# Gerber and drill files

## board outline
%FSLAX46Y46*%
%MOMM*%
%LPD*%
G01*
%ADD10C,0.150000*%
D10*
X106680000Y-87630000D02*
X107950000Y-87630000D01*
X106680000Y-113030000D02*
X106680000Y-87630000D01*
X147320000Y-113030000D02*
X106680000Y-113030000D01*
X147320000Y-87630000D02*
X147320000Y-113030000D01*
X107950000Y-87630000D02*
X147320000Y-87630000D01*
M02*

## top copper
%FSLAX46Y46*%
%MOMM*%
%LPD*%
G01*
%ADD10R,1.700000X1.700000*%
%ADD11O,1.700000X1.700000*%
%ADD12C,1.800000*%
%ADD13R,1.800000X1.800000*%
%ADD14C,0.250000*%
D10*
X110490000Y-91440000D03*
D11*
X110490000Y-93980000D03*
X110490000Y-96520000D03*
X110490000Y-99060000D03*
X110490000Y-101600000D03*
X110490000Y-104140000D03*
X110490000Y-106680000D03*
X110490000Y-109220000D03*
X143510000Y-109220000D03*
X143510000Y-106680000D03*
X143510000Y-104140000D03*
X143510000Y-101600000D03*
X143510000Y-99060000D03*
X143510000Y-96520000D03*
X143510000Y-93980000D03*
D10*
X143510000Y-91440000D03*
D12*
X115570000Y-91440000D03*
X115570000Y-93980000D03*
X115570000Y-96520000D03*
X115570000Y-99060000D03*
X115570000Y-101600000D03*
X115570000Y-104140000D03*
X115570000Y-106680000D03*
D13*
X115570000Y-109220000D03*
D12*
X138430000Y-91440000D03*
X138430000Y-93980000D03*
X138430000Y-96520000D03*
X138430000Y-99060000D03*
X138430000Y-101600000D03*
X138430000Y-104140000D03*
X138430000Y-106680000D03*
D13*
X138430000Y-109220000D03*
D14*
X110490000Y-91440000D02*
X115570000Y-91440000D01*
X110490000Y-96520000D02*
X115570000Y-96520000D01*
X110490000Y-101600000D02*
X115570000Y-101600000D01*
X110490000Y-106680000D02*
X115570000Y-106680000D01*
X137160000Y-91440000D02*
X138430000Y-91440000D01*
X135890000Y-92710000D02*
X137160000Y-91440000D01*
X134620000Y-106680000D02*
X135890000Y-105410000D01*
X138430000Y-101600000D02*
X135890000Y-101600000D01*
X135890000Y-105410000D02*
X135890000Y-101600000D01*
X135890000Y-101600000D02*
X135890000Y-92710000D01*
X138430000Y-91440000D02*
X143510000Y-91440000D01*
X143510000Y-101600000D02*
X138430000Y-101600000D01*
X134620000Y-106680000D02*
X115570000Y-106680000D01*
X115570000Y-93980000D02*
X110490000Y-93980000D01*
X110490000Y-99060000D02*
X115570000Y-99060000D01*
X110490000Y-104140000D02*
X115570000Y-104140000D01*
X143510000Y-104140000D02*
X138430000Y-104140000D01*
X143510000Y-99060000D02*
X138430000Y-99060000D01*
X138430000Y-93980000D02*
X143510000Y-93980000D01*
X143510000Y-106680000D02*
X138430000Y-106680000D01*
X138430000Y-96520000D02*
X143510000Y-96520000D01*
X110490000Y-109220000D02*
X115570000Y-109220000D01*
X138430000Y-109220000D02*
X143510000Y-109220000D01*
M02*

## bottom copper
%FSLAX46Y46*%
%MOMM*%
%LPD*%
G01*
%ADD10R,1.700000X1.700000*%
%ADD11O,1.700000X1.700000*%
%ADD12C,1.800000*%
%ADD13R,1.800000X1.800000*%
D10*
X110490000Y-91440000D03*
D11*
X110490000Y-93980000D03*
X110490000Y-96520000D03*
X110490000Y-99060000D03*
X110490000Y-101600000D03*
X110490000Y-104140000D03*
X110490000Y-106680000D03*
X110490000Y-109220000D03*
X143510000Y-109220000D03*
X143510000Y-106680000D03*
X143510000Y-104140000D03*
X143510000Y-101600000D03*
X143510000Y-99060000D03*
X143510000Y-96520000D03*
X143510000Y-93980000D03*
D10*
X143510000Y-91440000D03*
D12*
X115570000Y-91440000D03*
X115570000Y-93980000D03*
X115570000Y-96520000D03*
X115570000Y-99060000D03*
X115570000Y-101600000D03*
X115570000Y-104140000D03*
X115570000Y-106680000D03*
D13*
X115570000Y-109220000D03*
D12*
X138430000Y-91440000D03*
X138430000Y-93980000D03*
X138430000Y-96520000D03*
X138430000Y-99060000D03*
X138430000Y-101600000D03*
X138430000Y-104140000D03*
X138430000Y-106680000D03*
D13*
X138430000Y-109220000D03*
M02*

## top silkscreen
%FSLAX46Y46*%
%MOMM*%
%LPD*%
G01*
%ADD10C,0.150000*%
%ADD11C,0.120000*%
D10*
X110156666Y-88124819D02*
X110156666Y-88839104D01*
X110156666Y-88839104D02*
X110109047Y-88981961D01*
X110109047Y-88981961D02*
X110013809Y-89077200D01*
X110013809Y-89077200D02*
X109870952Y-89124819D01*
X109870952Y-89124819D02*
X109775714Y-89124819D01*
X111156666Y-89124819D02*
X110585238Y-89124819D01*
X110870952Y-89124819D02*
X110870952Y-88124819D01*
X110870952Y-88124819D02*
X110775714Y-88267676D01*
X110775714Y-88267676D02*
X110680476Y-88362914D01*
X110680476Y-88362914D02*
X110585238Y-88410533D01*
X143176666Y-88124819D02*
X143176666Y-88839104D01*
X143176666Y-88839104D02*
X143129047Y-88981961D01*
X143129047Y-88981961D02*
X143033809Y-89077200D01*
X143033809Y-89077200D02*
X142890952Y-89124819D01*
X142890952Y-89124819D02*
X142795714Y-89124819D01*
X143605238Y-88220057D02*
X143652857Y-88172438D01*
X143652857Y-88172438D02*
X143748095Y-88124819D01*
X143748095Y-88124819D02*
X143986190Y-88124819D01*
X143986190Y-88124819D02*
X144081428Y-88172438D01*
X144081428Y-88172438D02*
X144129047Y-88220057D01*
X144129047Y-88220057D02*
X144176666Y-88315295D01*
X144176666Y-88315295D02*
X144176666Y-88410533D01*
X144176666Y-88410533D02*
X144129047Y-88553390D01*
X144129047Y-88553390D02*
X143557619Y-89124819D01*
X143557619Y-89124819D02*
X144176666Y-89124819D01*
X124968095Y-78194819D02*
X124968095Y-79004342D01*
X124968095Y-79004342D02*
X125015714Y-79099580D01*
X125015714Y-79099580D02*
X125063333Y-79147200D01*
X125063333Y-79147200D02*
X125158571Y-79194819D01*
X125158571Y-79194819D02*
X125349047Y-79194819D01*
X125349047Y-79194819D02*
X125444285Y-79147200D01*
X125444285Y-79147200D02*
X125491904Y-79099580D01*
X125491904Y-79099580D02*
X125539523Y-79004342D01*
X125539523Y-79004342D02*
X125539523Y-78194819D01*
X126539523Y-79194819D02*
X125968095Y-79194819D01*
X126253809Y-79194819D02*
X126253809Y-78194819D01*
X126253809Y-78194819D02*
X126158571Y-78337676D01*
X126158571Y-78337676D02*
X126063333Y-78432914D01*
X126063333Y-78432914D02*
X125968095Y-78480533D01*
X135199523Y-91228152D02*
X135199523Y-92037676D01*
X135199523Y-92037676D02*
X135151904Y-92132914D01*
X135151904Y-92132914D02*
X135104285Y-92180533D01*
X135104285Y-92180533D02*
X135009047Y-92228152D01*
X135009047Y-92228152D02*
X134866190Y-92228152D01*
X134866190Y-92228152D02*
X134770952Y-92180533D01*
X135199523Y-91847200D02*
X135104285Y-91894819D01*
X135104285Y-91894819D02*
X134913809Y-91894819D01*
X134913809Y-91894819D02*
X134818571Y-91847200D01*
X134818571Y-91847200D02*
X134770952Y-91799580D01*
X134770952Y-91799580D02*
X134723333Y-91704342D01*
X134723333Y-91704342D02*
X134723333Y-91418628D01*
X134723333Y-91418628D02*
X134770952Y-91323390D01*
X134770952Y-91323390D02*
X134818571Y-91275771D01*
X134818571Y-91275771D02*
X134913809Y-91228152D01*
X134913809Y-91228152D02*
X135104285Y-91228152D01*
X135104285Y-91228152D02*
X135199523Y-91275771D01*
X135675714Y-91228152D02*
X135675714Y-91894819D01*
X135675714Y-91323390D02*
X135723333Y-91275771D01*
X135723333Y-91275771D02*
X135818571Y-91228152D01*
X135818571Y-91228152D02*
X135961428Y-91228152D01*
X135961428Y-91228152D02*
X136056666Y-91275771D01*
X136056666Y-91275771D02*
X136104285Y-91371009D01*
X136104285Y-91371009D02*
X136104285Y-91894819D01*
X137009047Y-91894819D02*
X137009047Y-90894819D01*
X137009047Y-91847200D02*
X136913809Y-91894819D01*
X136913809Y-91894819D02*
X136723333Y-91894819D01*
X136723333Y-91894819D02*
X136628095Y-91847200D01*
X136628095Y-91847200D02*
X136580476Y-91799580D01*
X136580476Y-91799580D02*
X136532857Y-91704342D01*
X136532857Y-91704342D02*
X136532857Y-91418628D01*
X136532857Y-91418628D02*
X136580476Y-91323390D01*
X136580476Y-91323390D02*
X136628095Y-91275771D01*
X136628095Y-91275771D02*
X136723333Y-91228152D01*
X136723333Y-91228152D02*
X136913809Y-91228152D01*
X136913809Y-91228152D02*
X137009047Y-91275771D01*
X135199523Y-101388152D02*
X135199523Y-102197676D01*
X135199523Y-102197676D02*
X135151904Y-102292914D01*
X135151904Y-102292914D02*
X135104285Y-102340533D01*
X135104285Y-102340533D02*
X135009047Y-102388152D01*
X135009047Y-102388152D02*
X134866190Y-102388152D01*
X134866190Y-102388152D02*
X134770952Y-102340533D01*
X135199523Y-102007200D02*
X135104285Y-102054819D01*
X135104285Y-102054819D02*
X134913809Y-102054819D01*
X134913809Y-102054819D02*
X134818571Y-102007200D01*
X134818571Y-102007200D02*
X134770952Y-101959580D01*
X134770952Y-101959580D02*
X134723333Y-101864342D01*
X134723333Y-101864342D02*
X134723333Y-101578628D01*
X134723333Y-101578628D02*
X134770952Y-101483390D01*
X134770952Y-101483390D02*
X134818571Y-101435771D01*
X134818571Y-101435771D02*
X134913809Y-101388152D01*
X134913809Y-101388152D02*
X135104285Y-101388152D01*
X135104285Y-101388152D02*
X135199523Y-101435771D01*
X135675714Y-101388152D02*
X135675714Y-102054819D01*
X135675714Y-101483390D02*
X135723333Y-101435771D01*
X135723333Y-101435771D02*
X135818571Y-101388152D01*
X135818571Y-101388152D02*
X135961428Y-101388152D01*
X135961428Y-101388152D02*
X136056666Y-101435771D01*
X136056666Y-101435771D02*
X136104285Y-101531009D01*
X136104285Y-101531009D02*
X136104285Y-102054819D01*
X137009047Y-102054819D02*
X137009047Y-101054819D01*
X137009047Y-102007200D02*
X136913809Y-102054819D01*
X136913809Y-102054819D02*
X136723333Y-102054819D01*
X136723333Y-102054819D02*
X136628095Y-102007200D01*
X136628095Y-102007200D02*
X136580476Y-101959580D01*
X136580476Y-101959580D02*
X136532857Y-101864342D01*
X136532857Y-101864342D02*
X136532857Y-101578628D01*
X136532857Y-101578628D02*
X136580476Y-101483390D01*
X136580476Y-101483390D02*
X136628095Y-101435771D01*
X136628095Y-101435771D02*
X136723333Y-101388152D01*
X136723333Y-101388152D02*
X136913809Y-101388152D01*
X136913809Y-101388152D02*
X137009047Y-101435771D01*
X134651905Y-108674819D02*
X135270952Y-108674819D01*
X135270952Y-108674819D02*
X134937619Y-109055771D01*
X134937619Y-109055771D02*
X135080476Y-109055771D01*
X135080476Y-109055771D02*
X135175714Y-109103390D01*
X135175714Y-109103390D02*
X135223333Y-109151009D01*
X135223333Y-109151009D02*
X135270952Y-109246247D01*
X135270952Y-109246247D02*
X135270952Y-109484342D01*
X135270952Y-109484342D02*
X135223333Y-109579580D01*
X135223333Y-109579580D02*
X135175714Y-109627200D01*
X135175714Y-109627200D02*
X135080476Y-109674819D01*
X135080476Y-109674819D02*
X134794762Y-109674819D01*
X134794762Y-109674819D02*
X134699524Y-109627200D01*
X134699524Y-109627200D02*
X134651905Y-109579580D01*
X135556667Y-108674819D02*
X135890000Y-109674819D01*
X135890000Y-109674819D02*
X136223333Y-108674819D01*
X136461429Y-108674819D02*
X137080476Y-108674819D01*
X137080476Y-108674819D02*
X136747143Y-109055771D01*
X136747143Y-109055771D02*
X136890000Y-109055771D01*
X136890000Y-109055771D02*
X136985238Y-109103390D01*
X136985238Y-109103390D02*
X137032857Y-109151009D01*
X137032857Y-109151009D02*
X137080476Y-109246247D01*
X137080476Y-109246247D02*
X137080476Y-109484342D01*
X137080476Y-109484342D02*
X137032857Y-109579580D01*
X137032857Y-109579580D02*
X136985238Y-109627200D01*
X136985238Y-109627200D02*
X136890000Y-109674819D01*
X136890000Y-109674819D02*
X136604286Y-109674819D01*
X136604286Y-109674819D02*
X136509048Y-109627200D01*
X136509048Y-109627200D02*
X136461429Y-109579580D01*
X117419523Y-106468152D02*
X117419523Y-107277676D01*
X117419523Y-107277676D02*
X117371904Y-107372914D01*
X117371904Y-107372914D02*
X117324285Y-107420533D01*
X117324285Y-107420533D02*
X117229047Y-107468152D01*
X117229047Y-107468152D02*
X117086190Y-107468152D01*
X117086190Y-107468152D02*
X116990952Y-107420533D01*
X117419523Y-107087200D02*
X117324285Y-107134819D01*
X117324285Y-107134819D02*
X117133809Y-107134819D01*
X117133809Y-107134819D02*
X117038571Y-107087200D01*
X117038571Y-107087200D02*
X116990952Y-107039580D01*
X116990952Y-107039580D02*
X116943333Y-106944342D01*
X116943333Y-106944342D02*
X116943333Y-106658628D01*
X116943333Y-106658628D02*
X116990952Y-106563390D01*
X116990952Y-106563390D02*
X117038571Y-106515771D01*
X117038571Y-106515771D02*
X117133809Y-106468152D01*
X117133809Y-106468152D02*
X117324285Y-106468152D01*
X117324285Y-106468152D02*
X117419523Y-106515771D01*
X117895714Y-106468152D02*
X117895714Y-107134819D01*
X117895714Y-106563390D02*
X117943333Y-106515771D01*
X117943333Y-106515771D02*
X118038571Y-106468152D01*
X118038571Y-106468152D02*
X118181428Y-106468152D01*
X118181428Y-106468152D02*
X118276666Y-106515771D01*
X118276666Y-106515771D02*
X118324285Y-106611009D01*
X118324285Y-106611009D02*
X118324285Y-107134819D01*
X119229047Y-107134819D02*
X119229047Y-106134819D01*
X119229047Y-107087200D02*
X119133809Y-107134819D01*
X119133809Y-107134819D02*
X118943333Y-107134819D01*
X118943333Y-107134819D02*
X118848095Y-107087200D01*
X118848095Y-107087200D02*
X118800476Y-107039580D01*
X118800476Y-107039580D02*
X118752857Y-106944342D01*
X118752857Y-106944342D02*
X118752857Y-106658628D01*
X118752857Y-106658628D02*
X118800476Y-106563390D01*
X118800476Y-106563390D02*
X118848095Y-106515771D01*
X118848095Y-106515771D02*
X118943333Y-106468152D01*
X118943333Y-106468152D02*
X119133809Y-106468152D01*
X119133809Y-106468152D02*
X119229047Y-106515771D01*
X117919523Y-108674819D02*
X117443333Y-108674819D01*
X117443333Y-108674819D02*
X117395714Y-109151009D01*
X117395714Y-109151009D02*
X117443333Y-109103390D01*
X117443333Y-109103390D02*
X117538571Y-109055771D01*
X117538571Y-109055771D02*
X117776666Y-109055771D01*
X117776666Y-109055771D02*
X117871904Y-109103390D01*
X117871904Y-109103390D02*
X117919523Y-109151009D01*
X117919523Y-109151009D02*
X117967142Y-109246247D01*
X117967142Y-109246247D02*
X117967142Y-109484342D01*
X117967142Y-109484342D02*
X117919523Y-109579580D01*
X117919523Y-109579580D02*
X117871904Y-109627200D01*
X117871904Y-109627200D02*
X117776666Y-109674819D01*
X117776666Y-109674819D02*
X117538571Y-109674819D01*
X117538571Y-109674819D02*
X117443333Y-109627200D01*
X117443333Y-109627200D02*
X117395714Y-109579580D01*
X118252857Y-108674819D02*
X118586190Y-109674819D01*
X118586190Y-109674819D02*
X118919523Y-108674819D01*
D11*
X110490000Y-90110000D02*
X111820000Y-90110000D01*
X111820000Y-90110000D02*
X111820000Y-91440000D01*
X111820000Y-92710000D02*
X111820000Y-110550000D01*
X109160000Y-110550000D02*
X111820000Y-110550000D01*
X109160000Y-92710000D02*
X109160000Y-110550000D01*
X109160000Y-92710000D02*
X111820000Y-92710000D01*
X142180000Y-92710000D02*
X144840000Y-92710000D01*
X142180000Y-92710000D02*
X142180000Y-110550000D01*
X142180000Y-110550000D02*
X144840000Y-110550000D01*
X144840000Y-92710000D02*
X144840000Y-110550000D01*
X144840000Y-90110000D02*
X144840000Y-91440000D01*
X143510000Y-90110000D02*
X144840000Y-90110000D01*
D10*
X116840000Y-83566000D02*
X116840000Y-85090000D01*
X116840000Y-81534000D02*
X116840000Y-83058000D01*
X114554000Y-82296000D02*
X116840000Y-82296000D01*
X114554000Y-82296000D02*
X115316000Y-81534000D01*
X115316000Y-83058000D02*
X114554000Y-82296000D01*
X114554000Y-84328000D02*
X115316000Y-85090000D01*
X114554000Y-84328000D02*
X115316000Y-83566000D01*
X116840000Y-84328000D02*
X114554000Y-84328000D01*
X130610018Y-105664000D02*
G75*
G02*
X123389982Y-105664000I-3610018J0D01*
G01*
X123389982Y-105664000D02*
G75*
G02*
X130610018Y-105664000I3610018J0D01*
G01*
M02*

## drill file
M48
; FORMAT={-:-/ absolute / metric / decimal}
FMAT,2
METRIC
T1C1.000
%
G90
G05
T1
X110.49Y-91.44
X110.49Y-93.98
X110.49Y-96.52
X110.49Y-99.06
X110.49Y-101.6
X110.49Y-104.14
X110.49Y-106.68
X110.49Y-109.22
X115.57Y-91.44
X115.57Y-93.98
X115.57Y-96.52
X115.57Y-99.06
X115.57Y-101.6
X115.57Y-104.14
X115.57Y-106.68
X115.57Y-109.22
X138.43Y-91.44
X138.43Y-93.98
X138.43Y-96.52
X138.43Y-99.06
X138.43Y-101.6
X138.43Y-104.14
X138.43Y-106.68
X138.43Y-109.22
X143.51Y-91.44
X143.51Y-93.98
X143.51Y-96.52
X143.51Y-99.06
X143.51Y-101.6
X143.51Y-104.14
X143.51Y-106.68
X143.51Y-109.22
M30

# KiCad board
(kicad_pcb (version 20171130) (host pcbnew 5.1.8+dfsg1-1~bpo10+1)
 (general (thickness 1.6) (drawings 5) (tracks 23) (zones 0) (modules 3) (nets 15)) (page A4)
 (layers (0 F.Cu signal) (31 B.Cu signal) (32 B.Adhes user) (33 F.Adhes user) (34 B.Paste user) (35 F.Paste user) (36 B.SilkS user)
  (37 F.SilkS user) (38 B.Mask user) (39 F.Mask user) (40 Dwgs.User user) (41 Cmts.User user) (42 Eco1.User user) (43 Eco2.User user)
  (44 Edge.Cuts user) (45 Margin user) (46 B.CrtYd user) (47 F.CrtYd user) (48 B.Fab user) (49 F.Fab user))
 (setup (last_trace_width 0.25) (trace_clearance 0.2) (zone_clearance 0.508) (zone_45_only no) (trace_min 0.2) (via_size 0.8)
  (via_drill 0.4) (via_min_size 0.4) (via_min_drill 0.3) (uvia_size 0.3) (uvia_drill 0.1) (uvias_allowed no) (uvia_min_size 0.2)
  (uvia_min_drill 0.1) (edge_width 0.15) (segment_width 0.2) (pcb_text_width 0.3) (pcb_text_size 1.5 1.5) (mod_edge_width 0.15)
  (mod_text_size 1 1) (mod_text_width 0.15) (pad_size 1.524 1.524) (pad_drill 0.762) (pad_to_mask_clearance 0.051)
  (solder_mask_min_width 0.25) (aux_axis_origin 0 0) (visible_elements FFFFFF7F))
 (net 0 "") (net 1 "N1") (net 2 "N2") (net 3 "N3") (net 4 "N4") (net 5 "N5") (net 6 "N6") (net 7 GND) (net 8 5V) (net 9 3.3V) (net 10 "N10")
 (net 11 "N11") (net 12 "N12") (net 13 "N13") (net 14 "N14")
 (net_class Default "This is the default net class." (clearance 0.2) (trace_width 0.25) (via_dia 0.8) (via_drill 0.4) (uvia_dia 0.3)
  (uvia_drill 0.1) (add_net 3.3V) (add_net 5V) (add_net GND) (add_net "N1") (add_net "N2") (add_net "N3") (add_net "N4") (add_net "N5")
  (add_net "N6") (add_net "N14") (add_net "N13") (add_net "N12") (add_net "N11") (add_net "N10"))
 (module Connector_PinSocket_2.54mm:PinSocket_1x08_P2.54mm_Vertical (layer F.Cu) (at 110.49 91.44)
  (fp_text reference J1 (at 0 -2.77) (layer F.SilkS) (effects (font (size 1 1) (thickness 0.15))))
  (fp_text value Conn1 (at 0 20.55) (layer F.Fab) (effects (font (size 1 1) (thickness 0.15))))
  (fp_line (start 0 -1.33) (end 1.33 -1.33) (layer F.SilkS) (width 0.12))
  (fp_line (start 1.33 -1.33) (end 1.33 0) (layer F.SilkS) (width 0.12))
  (fp_line (start 1.33 1.27) (end 1.33 19.11) (layer F.SilkS) (width 0.12))
  (fp_line (start -1.33 19.11) (end 1.33 19.11) (layer F.SilkS) (width 0.12))
  (fp_line (start -1.33 1.27) (end -1.33 19.11) (layer F.SilkS) (width 0.12))
  (fp_line (start -1.33 1.27) (end 1.33 1.27) (layer F.SilkS) (width 0.12))
  (pad 1 thru_hole rect (at 0 0) (size 1.7 1.7) (drill 1) (layers *.Cu *.Mask) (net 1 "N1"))
  (pad 2 thru_hole oval (at 0 2.54) (size 1.7 1.7) (drill 1) (layers *.Cu *.Mask) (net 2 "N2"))
  (pad 3 thru_hole oval (at 0 5.08) (size 1.7 1.7) (drill 1) (layers *.Cu *.Mask) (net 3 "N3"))
  (pad 4 thru_hole oval (at 0 7.62) (size 1.7 1.7) (drill 1) (layers *.Cu *.Mask) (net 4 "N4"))
  (pad 5 thru_hole oval (at 0 10.16) (size 1.7 1.7) (drill 1) (layers *.Cu *.Mask) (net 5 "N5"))
  (pad 6 thru_hole oval (at 0 12.7) (size 1.7 1.7) (drill 1) (layers *.Cu *.Mask) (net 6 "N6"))
  (pad 7 thru_hole oval (at 0 15.24) (size 1.7 1.7) (drill 1) (layers *.Cu *.Mask) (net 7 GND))
  (pad 8 thru_hole oval (at 0 17.78) (size 1.7 1.7) (drill 1) (layers *.Cu *.Mask) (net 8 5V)))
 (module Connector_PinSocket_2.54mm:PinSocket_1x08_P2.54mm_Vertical (layer F.Cu) (at 143.51 91.44)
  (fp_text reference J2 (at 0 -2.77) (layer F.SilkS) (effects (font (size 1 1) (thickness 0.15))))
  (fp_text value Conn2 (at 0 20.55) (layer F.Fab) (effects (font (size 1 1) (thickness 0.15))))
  (fp_line (start -1.33 1.27) (end 1.33 1.27) (layer F.SilkS) (width 0.12))
  (fp_line (start -1.33 1.27) (end -1.33 19.11) (layer F.SilkS) (width 0.12))
  (fp_line (start -1.33 19.11) (end 1.33 19.11) (layer F.SilkS) (width 0.12))
  (fp_line (start 1.33 1.27) (end 1.33 19.11) (layer F.SilkS) (width 0.12))
  (fp_line (start 1.33 -1.33) (end 1.33 0) (layer F.SilkS) (width 0.12))
  (fp_line (start 0 -1.33) (end 1.33 -1.33) (layer F.SilkS) (width 0.12))
  (pad 8 thru_hole oval (at 0 17.78) (size 1.7 1.7) (drill 1) (layers *.Cu *.Mask) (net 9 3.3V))
  (pad 7 thru_hole oval (at 0 15.24) (size 1.7 1.7) (drill 1) (layers *.Cu *.Mask) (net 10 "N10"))
  (pad 6 thru_hole oval (at 0 12.7) (size 1.7 1.7) (drill 1) (layers *.Cu *.Mask) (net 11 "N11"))
  (pad 5 thru_hole oval (at 0 10.16) (size 1.7 1.7) (drill 1) (layers *.Cu *.Mask) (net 7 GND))
  (pad 4 thru_hole oval (at 0 7.62) (size 1.7 1.7) (drill 1) (layers *.Cu *.Mask) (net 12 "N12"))
  (pad 3 thru_hole oval (at 0 5.08) (size 1.7 1.7) (drill 1) (layers *.Cu *.Mask) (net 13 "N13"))
  (pad 2 thru_hole oval (at 0 2.54) (size 1.7 1.7) (drill 1) (layers *.Cu *.Mask) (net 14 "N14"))
  (pad 1 thru_hole rect (at 0 0) (size 1.7 1.7) (drill 1) (layers *.Cu *.Mask) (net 7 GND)))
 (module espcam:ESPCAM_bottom (layer F.Cu) (at 125.73 88.9)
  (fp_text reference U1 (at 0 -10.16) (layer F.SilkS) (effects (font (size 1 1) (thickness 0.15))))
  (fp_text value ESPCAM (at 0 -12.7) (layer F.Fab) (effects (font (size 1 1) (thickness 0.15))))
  (fp_line (start -8.89 -5.334) (end -8.89 -3.81) (layer F.SilkS) (width 0.15))
  (fp_line (start -8.89 -7.366) (end -8.89 -5.842) (layer F.SilkS) (width 0.15))
  (fp_line (start -11.176 -6.604) (end -8.89 -6.604) (layer F.SilkS) (width 0.15))
  (fp_line (start -11.176 -6.604) (end -10.414 -7.366) (layer F.SilkS) (width 0.15))
  (fp_line (start -10.414 -5.842) (end -11.176 -6.604) (layer F.SilkS) (width 0.15))
  (fp_line (start -11.176 -4.572) (end -10.414 -3.81) (layer F.SilkS) (width 0.15))
  (fp_line (start -11.176 -4.572) (end -10.414 -5.334) (layer F.SilkS) (width 0.15))
  (fp_line (start -8.89 -4.572) (end -11.176 -4.572) (layer F.SilkS) (width 0.15))
  (fp_circle (center 1.27 16.764) (end 3.556 19.558) (layer F.SilkS) (width 0.15))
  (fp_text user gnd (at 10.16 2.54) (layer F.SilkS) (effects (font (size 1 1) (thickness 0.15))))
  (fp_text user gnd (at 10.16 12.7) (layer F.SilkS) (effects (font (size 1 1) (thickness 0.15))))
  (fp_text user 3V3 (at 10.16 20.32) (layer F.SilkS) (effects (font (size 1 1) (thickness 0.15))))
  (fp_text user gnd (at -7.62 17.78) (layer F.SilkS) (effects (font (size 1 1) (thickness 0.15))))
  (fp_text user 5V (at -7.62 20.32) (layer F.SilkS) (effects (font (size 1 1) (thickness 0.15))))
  (pad 1 thru_hole circle (at -10.16 2.54) (size 1.8 1.8) (drill 1) (layers *.Cu *.Mask) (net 1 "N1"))
  (pad 2 thru_hole circle (at -10.16 5.08) (size 1.8 1.8) (drill 1) (layers *.Cu *.Mask) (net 2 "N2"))
  (pad 3 thru_hole circle (at -10.16 7.62) (size 1.8 1.8) (drill 1) (layers *.Cu *.Mask) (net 3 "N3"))
  (pad 4 thru_hole circle (at -10.16 10.16) (size 1.8 1.8) (drill 1) (layers *.Cu *.Mask) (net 4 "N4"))
  (pad 5 thru_hole circle (at -10.16 12.7) (size 1.8 1.8) (drill 1) (layers *.Cu *.Mask) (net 5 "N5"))
  (pad 6 thru_hole circle (at -10.16 15.24) (size 1.8 1.8) (drill 1) (layers *.Cu *.Mask) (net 6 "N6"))
  (pad 7 thru_hole circle (at -10.16 17.78) (size 1.8 1.8) (drill 1) (layers *.Cu *.Mask) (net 7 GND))
  (pad 8 thru_hole rect (at -10.16 20.32) (size 1.8 1.8) (drill 1) (layers *.Cu *.Mask) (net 8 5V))
  (pad 9 thru_hole circle (at 12.7 2.54) (size 1.8 1.8) (drill 1) (layers *.Cu *.Mask) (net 7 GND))
  (pad 10 thru_hole circle (at 12.7 5.08) (size 1.8 1.8) (drill 1) (layers *.Cu *.Mask) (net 14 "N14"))
  (pad 11 thru_hole circle (at 12.7 7.62) (size 1.8 1.8) (drill 1) (layers *.Cu *.Mask) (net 13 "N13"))
  (pad 12 thru_hole circle (at 12.7 10.16) (size 1.8 1.8) (drill 1) (layers *.Cu *.Mask) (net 12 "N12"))
  (pad 13 thru_hole circle (at 12.7 12.7) (size 1.8 1.8) (drill 1) (layers *.Cu *.Mask) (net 7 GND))
  (pad 14 thru_hole circle (at 12.7 15.24) (size 1.8 1.8) (drill 1) (layers *.Cu *.Mask) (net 11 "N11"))
  (pad 15 thru_hole circle (at 12.7 17.78) (size 1.8 1.8) (drill 1) (layers *.Cu *.Mask) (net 10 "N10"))
  (pad 16 thru_hole rect (at 12.7 20.32) (size 1.8 1.8) (drill 1) (layers *.Cu *.Mask) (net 9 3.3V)))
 (gr_line (start 106.68 87.63) (end 107.95 87.63) (layer Edge.Cuts) (width 0.15))
 (gr_line (start 106.68 113.03) (end 106.68 87.63) (layer Edge.Cuts) (width 0.15))
 (gr_line (start 147.32 113.03) (end 106.68 113.03) (layer Edge.Cuts) (width 0.15))
 (gr_line (start 147.32 87.63) (end 147.32 113.03) (layer Edge.Cuts) (width 0.15))
 (gr_line (start 107.95 87.63) (end 147.32 87.63) (layer Edge.Cuts) (width 0.15))
 (segment (start 110.49 91.44) (end 115.57 91.44) (width 0.25) (layer F.Cu) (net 1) (status 10))
 (segment (start 110.49 96.52) (end 115.57 96.52) (width 0.25) (layer F.Cu) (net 3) (status 10))
 (segment (start 110.49 101.6) (end 115.57 101.6) (width 0.25) (layer F.Cu) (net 5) (status 10))
 (segment (start 110.49 106.68) (end 115.57 106.68) (width 0.25) (layer F.Cu) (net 7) (status 10))
 (segment (start 137.16 91.44) (end 138.43 91.44) (width 0.25) (layer F.Cu) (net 7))
 (segment (start 135.89 92.71) (end 137.16 91.44) (width 0.25) (layer F.Cu) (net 7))
 (segment (start 134.62 106.68) (end 135.89 105.41) (width 0.25) (layer F.Cu) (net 7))
 (segment (start 138.43 101.6) (end 135.89 101.6) (width 0.25) (layer F.Cu) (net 7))
 (segment (start 135.89 105.41) (end 135.89 101.6) (width 0.25) (layer F.Cu) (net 7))
 (segment (start 135.89 101.6) (end 135.89 92.71) (width 0.25) (layer F.Cu) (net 7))
 (segment (start 138.43 91.44) (end 143.51 91.44) (width 0.25) (layer F.Cu) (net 7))
 (segment (start 143.51 101.6) (end 138.43 101.6) (width 0.25) (layer F.Cu) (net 7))
 (segment (start 134.62 106.68) (end 115.57 106.68) (width 0.25) (layer F.Cu) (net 7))
 (segment (start 115.57 93.98) (end 110.49 93.98) (width 0.25) (layer F.Cu) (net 2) (status 20))
 (segment (start 110.49 99.06) (end 115.57 99.06) (width 0.25) (layer F.Cu) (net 4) (status 10))
 (segment (start 110.49 104.14) (end 115.57 104.14) (width 0.25) (layer F.Cu) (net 6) (status 10))
 (segment (start 143.51 104.14) (end 138.43 104.14) (width 0.25) (layer F.Cu) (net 11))
 (segment (start 143.51 99.06) (end 138.43 99.06) (width 0.25) (layer F.Cu) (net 12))
 (segment (start 138.43 93.98) (end 143.51 93.98) (width 0.25) (layer F.Cu) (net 14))
 (segment (start 143.51 106.68) (end 138.43 106.68) (width 0.25) (layer F.Cu) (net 10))
 (segment (start 138.43 96.52) (end 143.51 96.52) (width 0.25) (layer F.Cu) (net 13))
 (segment (start 110.49 109.22) (end 115.57 109.22) (width 0.25) (layer F.Cu) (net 8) (status 10))
 (segment (start 138.43 109.22) (end 143.51 109.22) (width 0.25) (layer F.Cu) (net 9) (status 20)))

